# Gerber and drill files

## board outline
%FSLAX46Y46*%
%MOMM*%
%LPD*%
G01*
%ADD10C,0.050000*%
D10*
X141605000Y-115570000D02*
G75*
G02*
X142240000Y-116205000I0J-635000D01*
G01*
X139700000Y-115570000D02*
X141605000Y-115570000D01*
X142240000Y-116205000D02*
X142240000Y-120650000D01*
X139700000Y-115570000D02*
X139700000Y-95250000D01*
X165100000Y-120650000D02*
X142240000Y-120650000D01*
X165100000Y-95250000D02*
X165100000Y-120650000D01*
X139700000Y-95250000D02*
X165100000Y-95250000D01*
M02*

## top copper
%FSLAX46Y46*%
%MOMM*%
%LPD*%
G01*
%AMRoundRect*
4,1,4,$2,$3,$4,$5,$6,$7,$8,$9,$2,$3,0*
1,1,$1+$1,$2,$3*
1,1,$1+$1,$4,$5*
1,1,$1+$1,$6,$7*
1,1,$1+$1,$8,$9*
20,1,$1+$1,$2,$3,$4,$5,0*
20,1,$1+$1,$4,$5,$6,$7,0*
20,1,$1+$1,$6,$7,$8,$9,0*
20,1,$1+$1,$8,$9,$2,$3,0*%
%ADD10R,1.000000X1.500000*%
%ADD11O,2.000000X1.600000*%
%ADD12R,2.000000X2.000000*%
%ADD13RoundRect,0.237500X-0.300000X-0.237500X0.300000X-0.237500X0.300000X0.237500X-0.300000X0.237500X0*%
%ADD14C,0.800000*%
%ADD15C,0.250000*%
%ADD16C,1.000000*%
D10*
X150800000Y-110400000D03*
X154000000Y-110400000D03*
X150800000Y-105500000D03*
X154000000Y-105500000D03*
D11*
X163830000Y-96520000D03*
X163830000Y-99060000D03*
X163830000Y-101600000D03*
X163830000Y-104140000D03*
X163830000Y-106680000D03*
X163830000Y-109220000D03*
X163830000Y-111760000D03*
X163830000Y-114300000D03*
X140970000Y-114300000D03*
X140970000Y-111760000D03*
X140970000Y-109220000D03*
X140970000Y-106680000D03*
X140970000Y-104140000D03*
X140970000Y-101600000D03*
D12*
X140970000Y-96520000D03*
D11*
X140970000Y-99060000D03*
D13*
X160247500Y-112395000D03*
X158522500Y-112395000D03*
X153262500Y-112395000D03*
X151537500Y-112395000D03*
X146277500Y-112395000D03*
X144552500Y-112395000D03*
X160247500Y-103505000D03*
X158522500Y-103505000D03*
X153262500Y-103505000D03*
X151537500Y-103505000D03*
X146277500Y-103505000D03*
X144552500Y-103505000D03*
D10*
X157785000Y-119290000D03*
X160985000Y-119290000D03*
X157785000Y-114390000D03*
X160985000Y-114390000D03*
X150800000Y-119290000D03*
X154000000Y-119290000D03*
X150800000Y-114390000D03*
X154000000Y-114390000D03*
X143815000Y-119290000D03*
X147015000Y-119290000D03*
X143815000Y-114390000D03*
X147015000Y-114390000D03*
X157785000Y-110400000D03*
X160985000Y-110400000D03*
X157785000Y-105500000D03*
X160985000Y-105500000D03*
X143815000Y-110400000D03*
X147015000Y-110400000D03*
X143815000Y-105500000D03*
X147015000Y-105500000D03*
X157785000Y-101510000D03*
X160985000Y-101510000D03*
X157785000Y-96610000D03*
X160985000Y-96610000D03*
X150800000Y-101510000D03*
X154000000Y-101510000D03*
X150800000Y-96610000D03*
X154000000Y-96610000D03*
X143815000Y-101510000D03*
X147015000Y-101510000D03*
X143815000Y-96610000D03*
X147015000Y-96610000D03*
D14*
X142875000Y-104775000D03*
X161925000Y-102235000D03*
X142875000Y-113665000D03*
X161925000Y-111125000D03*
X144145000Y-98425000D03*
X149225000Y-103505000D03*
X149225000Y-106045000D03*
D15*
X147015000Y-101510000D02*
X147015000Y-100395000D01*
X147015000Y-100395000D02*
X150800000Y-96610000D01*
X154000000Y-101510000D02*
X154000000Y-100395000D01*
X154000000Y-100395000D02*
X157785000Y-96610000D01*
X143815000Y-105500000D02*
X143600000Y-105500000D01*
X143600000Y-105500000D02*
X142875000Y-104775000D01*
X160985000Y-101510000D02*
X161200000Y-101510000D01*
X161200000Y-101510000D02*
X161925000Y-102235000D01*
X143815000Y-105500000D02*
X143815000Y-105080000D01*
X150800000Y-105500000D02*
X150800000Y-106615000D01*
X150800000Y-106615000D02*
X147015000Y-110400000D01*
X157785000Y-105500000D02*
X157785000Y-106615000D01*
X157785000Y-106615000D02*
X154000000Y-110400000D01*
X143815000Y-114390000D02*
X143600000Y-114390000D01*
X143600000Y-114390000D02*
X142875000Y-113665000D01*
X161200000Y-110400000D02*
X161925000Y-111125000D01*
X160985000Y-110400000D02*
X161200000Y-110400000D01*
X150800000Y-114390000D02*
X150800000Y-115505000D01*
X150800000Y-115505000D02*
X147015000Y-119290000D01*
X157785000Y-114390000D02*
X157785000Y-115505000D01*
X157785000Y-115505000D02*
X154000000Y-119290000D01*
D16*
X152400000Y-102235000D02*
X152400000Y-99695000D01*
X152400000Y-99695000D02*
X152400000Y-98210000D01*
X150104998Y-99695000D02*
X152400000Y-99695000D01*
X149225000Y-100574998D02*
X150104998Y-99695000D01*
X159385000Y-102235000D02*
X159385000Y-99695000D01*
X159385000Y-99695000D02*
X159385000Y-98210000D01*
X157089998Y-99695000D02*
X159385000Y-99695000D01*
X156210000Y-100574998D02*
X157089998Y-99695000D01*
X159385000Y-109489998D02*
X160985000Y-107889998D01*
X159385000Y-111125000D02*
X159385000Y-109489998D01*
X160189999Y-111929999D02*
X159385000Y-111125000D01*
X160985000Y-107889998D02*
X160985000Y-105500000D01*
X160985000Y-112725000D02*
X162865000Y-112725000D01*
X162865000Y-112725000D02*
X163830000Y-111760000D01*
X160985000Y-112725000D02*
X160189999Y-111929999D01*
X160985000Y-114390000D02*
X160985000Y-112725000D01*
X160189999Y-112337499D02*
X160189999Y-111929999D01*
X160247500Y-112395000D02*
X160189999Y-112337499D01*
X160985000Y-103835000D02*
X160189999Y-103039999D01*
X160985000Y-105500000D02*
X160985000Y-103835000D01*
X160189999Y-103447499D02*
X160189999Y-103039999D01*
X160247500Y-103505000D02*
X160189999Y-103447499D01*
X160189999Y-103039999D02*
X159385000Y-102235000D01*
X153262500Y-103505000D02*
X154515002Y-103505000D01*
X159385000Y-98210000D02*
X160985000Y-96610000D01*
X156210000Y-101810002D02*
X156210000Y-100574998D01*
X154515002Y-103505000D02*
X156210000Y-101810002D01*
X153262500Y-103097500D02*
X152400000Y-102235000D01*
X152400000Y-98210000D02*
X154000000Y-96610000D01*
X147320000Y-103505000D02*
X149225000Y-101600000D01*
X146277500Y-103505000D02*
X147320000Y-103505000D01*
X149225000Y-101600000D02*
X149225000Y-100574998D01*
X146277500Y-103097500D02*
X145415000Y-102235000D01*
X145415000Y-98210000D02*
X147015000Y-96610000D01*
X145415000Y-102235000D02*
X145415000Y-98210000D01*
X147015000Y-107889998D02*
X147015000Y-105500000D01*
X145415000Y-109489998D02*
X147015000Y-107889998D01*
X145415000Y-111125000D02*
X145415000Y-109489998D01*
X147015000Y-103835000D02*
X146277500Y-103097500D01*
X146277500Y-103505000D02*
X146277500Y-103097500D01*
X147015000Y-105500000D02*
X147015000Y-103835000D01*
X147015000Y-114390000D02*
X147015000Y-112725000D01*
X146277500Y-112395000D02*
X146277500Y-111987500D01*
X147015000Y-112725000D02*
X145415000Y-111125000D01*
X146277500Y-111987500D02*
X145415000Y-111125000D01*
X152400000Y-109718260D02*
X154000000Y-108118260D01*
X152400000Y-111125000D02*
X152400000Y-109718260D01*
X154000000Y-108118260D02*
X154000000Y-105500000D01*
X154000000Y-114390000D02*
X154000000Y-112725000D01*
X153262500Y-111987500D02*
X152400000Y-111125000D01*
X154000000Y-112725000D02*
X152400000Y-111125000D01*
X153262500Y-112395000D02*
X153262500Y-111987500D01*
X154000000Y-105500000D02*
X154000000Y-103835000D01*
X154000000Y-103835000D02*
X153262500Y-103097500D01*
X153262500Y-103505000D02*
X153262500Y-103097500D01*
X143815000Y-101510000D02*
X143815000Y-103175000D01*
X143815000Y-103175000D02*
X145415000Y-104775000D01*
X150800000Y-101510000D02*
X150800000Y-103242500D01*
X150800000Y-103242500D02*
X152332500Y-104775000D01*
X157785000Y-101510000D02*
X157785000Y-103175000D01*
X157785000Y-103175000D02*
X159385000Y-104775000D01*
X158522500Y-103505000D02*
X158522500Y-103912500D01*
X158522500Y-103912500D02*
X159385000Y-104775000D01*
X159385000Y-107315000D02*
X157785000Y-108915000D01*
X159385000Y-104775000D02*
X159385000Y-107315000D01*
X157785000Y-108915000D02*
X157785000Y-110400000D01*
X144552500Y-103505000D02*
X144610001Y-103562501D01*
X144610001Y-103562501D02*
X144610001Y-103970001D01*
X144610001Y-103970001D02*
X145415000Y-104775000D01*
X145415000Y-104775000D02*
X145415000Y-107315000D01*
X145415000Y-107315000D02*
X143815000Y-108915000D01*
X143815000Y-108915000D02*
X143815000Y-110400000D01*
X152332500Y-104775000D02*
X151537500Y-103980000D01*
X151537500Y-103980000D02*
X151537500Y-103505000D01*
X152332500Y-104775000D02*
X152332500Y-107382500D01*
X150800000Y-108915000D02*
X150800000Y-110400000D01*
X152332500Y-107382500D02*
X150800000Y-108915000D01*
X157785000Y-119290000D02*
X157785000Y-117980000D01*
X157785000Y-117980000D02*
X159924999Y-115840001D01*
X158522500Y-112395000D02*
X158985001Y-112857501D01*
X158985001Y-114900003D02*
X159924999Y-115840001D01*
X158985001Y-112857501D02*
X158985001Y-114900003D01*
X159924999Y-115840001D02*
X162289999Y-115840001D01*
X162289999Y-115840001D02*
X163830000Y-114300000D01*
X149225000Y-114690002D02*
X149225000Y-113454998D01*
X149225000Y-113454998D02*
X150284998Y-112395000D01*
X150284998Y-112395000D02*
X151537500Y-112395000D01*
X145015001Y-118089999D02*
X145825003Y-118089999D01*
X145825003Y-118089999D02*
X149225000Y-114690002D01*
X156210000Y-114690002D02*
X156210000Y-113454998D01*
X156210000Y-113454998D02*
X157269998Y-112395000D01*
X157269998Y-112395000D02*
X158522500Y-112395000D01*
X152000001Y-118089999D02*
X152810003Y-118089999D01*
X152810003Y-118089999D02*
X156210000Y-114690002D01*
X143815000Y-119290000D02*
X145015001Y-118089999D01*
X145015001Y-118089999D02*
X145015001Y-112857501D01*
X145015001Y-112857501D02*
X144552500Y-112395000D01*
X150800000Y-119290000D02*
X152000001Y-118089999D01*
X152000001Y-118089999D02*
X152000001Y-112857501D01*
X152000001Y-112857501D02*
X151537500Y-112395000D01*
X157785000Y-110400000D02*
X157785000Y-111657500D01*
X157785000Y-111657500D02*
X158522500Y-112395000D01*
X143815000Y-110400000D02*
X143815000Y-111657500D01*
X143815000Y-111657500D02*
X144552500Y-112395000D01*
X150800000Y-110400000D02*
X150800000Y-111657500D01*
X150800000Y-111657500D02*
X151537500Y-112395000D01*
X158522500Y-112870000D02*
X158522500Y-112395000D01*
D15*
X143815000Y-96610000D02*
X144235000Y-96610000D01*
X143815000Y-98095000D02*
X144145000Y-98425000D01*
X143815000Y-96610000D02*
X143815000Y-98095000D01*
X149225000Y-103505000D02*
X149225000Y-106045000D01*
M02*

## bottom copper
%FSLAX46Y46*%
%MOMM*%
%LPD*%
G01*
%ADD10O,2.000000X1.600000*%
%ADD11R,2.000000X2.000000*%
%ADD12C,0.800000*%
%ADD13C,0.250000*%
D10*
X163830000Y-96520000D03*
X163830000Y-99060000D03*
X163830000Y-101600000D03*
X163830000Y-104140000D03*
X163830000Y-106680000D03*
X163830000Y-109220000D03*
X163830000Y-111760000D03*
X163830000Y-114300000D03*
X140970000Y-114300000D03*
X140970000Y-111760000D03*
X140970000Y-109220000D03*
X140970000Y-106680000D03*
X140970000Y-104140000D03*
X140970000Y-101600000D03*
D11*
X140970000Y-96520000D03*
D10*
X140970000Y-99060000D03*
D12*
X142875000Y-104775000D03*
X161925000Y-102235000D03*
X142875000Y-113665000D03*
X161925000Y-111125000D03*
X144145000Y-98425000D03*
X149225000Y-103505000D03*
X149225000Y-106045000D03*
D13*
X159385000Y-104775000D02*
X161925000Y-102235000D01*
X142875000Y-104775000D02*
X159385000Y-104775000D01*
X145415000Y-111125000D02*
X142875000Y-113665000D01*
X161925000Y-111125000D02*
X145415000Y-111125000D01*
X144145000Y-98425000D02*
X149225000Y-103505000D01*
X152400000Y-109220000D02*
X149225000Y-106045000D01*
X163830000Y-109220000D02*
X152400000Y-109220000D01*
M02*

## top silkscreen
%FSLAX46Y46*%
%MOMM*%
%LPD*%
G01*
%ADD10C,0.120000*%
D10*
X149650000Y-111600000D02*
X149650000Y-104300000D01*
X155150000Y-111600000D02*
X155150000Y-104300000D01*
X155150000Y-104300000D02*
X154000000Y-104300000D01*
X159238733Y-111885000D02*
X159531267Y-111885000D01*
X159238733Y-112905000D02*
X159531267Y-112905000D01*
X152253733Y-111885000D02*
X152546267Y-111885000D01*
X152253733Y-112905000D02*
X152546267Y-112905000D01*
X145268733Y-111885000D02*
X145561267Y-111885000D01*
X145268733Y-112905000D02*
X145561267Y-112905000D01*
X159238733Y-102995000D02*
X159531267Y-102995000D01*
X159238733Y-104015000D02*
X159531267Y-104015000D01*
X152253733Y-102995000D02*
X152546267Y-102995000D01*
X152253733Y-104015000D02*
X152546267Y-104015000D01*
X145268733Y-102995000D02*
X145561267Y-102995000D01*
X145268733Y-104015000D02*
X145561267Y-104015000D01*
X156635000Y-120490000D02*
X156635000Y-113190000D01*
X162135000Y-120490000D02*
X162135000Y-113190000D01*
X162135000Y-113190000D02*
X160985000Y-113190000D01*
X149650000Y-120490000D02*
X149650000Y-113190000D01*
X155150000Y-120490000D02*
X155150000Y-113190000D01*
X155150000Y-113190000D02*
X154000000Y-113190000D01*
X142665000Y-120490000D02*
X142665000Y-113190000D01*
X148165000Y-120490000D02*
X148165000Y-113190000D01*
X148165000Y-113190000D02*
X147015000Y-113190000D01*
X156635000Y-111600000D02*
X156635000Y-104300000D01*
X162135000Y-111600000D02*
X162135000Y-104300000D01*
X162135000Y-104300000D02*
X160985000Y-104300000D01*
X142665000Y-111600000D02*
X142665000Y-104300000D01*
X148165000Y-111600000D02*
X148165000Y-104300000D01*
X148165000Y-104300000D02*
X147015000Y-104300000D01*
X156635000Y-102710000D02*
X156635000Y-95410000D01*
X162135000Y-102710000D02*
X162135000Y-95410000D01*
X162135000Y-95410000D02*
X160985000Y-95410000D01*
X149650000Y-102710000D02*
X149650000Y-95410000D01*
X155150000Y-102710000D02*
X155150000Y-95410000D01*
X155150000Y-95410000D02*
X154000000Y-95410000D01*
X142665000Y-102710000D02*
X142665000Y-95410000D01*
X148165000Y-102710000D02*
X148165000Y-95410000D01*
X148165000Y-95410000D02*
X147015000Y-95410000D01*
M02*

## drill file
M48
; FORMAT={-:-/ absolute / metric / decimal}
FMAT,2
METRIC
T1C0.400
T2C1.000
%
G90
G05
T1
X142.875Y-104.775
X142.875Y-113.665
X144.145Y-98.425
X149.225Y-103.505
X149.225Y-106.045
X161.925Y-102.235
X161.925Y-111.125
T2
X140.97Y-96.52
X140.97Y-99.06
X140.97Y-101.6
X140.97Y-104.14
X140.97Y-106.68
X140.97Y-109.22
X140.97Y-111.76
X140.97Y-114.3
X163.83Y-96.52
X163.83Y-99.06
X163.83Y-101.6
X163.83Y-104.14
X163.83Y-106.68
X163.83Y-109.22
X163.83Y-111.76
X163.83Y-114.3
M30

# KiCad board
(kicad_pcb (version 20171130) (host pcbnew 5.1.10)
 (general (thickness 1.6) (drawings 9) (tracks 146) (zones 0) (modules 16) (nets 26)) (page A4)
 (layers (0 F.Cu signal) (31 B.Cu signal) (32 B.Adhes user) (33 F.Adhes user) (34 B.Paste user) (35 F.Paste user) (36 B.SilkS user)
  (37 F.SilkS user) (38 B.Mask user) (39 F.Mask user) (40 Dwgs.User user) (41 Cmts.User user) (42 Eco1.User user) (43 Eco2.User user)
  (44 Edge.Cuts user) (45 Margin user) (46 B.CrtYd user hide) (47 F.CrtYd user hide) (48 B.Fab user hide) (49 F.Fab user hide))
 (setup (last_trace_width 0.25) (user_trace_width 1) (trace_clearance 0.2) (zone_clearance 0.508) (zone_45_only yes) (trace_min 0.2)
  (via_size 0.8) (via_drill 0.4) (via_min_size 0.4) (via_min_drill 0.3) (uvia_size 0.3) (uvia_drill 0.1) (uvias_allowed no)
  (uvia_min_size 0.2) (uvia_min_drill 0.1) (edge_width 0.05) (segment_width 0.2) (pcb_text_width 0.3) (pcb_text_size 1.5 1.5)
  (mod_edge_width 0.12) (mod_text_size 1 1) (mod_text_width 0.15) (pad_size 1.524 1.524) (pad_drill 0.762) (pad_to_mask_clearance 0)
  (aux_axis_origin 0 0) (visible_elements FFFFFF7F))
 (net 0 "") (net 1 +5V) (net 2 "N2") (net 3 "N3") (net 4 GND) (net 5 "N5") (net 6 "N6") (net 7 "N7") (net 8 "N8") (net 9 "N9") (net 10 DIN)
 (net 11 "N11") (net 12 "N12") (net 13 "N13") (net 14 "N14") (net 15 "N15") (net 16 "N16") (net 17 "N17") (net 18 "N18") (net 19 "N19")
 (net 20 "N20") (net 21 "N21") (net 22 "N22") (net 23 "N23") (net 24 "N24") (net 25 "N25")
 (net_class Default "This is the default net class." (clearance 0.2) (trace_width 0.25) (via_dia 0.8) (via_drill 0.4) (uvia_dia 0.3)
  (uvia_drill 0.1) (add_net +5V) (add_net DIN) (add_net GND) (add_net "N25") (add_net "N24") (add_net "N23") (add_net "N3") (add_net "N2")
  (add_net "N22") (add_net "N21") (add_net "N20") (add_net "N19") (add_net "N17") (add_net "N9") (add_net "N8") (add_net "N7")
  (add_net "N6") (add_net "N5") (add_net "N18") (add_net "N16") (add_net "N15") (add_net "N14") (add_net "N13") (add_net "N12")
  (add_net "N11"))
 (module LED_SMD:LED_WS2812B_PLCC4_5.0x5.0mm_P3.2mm (layer F.Cu) (at 152.4 107.95 90)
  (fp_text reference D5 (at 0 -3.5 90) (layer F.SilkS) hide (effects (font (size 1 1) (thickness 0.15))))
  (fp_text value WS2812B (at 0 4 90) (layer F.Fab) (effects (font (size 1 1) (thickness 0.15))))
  (fp_line (start -3.65 -2.75) (end 3.65 -2.75) (layer F.SilkS) (width 0.12))
  (fp_line (start -3.65 2.75) (end 3.65 2.75) (layer F.SilkS) (width 0.12))
  (fp_line (start 3.65 2.75) (end 3.65 1.6) (layer F.SilkS) (width 0.12))
  (pad 1 smd rect (at -2.45 -1.6 90) (size 1.5 1) (layers F.Cu F.Paste F.Mask) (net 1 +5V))
  (pad 2 smd rect (at -2.45 1.6 90) (size 1.5 1) (layers F.Cu F.Paste F.Mask) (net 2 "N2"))
  (pad 4 smd rect (at 2.45 -1.6 90) (size 1.5 1) (layers F.Cu F.Paste F.Mask) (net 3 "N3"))
  (pad 3 smd rect (at 2.45 1.6 90) (size 1.5 1) (layers F.Cu F.Paste F.Mask) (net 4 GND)))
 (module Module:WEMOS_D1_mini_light (layer F.Cu) (at 140.97 96.52)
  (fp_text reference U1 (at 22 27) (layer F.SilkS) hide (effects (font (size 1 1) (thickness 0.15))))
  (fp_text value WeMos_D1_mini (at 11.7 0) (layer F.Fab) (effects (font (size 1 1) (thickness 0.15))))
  (pad 16 thru_hole oval (at 22.86 0) (size 2 1.6) (drill 1) (layers *.Cu *.Mask) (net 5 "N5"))
  (pad 15 thru_hole oval (at 22.86 2.54) (size 2 1.6) (drill 1) (layers *.Cu *.Mask) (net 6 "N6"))
  (pad 14 thru_hole oval (at 22.86 5.08) (size 2 1.6) (drill 1) (layers *.Cu *.Mask) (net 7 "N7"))
  (pad 13 thru_hole oval (at 22.86 7.62) (size 2 1.6) (drill 1) (layers *.Cu *.Mask) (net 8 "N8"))
  (pad 12 thru_hole oval (at 22.86 10.16) (size 2 1.6) (drill 1) (layers *.Cu *.Mask) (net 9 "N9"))
  (pad 11 thru_hole oval (at 22.86 12.7) (size 2 1.6) (drill 1) (layers *.Cu *.Mask) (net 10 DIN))
  (pad 10 thru_hole oval (at 22.86 15.24) (size 2 1.6) (drill 1) (layers *.Cu *.Mask) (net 4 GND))
  (pad 9 thru_hole oval (at 22.86 17.78) (size 2 1.6) (drill 1) (layers *.Cu *.Mask) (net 1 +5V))
  (pad 8 thru_hole oval (at 0 17.78) (size 2 1.6) (drill 1) (layers *.Cu *.Mask) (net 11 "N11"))
  (pad 7 thru_hole oval (at 0 15.24) (size 2 1.6) (drill 1) (layers *.Cu *.Mask) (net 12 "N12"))
  (pad 6 thru_hole oval (at 0 12.7) (size 2 1.6) (drill 1) (layers *.Cu *.Mask) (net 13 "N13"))
  (pad 5 thru_hole oval (at 0 10.16) (size 2 1.6) (drill 1) (layers *.Cu *.Mask) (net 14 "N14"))
  (pad 4 thru_hole oval (at 0 7.62) (size 2 1.6) (drill 1) (layers *.Cu *.Mask) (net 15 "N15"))
  (pad 3 thru_hole oval (at 0 5.08) (size 2 1.6) (drill 1) (layers *.Cu *.Mask) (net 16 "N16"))
  (pad 1 thru_hole rect (at 0 0) (size 2 2) (drill 1) (layers *.Cu *.Mask) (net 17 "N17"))
  (pad 2 thru_hole oval (at 0 2.54) (size 2 1.6) (drill 1) (layers *.Cu *.Mask) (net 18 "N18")))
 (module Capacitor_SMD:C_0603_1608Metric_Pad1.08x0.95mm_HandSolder (layer F.Cu) (at 159.385 112.395)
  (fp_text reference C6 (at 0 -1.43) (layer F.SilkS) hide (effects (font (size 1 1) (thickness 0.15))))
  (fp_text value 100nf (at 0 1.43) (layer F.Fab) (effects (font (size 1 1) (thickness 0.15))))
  (fp_line (start -0.146267 -0.51) (end 0.146267 -0.51) (layer F.SilkS) (width 0.12))
  (fp_line (start -0.146267 0.51) (end 0.146267 0.51) (layer F.SilkS) (width 0.12))
  (pad 2 smd roundrect (at 0.8625 0) (size 1.075 0.95) (layers F.Cu F.Paste F.Mask) (roundrect_rratio 0.25) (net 4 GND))
  (pad 1 smd roundrect (at -0.8625 0) (size 1.075 0.95) (layers F.Cu F.Paste F.Mask) (roundrect_rratio 0.25) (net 1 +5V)))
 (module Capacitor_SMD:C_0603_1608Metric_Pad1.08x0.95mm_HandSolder (layer F.Cu) (at 152.4 112.395)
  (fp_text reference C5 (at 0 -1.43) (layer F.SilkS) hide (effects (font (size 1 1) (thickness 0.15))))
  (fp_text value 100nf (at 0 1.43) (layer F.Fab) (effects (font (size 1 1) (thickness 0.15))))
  (fp_line (start -0.146267 -0.51) (end 0.146267 -0.51) (layer F.SilkS) (width 0.12))
  (fp_line (start -0.146267 0.51) (end 0.146267 0.51) (layer F.SilkS) (width 0.12))
  (pad 2 smd roundrect (at 0.8625 0) (size 1.075 0.95) (layers F.Cu F.Paste F.Mask) (roundrect_rratio 0.25) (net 4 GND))
  (pad 1 smd roundrect (at -0.8625 0) (size 1.075 0.95) (layers F.Cu F.Paste F.Mask) (roundrect_rratio 0.25) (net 1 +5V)))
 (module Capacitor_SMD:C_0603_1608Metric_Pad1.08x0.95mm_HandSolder (layer F.Cu) (at 145.415 112.395)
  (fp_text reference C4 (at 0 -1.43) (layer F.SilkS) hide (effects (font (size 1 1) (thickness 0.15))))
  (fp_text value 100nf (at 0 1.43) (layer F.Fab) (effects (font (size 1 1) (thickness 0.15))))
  (fp_line (start -0.146267 -0.51) (end 0.146267 -0.51) (layer F.SilkS) (width 0.12))
  (fp_line (start -0.146267 0.51) (end 0.146267 0.51) (layer F.SilkS) (width 0.12))
  (pad 2 smd roundrect (at 0.8625 0) (size 1.075 0.95) (layers F.Cu F.Paste F.Mask) (roundrect_rratio 0.25) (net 4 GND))
  (pad 1 smd roundrect (at -0.8625 0) (size 1.075 0.95) (layers F.Cu F.Paste F.Mask) (roundrect_rratio 0.25) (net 1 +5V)))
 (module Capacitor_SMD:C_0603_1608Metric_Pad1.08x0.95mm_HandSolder (layer F.Cu) (at 159.385 103.505)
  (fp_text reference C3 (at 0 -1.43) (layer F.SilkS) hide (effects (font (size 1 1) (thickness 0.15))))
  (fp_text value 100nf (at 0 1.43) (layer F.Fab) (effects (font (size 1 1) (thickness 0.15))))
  (fp_line (start -0.146267 -0.51) (end 0.146267 -0.51) (layer F.SilkS) (width 0.12))
  (fp_line (start -0.146267 0.51) (end 0.146267 0.51) (layer F.SilkS) (width 0.12))
  (pad 2 smd roundrect (at 0.8625 0) (size 1.075 0.95) (layers F.Cu F.Paste F.Mask) (roundrect_rratio 0.25) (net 4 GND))
  (pad 1 smd roundrect (at -0.8625 0) (size 1.075 0.95) (layers F.Cu F.Paste F.Mask) (roundrect_rratio 0.25) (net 1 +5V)))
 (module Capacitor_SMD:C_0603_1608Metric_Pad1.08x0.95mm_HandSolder (layer F.Cu) (at 152.4 103.505)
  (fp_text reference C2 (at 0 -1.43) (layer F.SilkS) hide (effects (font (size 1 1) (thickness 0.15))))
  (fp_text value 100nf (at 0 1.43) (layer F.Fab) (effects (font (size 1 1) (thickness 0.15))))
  (fp_line (start -0.146267 -0.51) (end 0.146267 -0.51) (layer F.SilkS) (width 0.12))
  (fp_line (start -0.146267 0.51) (end 0.146267 0.51) (layer F.SilkS) (width 0.12))
  (pad 2 smd roundrect (at 0.8625 0) (size 1.075 0.95) (layers F.Cu F.Paste F.Mask) (roundrect_rratio 0.25) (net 4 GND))
  (pad 1 smd roundrect (at -0.8625 0) (size 1.075 0.95) (layers F.Cu F.Paste F.Mask) (roundrect_rratio 0.25) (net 1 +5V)))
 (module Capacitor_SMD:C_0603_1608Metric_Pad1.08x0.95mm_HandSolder (layer F.Cu) (at 145.415 103.505)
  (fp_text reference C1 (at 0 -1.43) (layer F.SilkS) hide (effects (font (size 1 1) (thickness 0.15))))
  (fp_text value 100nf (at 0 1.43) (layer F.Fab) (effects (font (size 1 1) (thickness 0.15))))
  (fp_line (start -0.146267 -0.51) (end 0.146267 -0.51) (layer F.SilkS) (width 0.12))
  (fp_line (start -0.146267 0.51) (end 0.146267 0.51) (layer F.SilkS) (width 0.12))
  (pad 2 smd roundrect (at 0.8625 0) (size 1.075 0.95) (layers F.Cu F.Paste F.Mask) (roundrect_rratio 0.25) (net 4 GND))
  (pad 1 smd roundrect (at -0.8625 0) (size 1.075 0.95) (layers F.Cu F.Paste F.Mask) (roundrect_rratio 0.25) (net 1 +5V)))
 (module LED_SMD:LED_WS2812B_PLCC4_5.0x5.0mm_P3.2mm (layer F.Cu) (at 159.385 116.84 90)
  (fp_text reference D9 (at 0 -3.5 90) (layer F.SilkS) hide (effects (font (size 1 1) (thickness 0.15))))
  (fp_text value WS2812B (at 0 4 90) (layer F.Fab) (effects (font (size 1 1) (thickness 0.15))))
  (fp_line (start -3.65 -2.75) (end 3.65 -2.75) (layer F.SilkS) (width 0.12))
  (fp_line (start -3.65 2.75) (end 3.65 2.75) (layer F.SilkS) (width 0.12))
  (fp_line (start 3.65 2.75) (end 3.65 1.6) (layer F.SilkS) (width 0.12))
  (pad 1 smd rect (at -2.45 -1.6 90) (size 1.5 1) (layers F.Cu F.Paste F.Mask) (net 1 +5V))
  (pad 2 smd rect (at -2.45 1.6 90) (size 1.5 1) (layers F.Cu F.Paste F.Mask) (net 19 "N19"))
  (pad 4 smd rect (at 2.45 -1.6 90) (size 1.5 1) (layers F.Cu F.Paste F.Mask) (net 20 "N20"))
  (pad 3 smd rect (at 2.45 1.6 90) (size 1.5 1) (layers F.Cu F.Paste F.Mask) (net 4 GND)))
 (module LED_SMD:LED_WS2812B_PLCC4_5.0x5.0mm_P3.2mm (layer F.Cu) (at 152.4 116.84 90)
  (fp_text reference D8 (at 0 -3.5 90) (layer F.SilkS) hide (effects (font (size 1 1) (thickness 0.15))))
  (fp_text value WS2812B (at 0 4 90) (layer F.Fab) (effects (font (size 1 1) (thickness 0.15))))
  (fp_line (start -3.65 -2.75) (end 3.65 -2.75) (layer F.SilkS) (width 0.12))
  (fp_line (start -3.65 2.75) (end 3.65 2.75) (layer F.SilkS) (width 0.12))
  (fp_line (start 3.65 2.75) (end 3.65 1.6) (layer F.SilkS) (width 0.12))
  (pad 1 smd rect (at -2.45 -1.6 90) (size 1.5 1) (layers F.Cu F.Paste F.Mask) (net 1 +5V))
  (pad 2 smd rect (at -2.45 1.6 90) (size 1.5 1) (layers F.Cu F.Paste F.Mask) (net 20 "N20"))
  (pad 4 smd rect (at 2.45 -1.6 90) (size 1.5 1) (layers F.Cu F.Paste F.Mask) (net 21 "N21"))
  (pad 3 smd rect (at 2.45 1.6 90) (size 1.5 1) (layers F.Cu F.Paste F.Mask) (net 4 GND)))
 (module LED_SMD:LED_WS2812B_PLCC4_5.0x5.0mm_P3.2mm (layer F.Cu) (at 145.415 116.84 90)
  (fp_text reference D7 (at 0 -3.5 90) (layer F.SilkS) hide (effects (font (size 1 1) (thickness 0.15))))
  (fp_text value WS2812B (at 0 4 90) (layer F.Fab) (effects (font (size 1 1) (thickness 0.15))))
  (fp_line (start -3.65 -2.75) (end 3.65 -2.75) (layer F.SilkS) (width 0.12))
  (fp_line (start -3.65 2.75) (end 3.65 2.75) (layer F.SilkS) (width 0.12))
  (fp_line (start 3.65 2.75) (end 3.65 1.6) (layer F.SilkS) (width 0.12))
  (pad 1 smd rect (at -2.45 -1.6 90) (size 1.5 1) (layers F.Cu F.Paste F.Mask) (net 1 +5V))
  (pad 2 smd rect (at -2.45 1.6 90) (size 1.5 1) (layers F.Cu F.Paste F.Mask) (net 21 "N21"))
  (pad 4 smd rect (at 2.45 -1.6 90) (size 1.5 1) (layers F.Cu F.Paste F.Mask) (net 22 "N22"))
  (pad 3 smd rect (at 2.45 1.6 90) (size 1.5 1) (layers F.Cu F.Paste F.Mask) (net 4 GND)))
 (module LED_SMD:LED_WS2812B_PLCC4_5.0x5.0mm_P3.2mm (layer F.Cu) (at 159.385 107.95 90)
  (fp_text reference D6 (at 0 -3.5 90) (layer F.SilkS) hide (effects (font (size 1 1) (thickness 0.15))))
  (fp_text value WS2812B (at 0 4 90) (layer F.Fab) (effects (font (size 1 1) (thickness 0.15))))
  (fp_line (start -3.65 -2.75) (end 3.65 -2.75) (layer F.SilkS) (width 0.12))
  (fp_line (start -3.65 2.75) (end 3.65 2.75) (layer F.SilkS) (width 0.12))
  (fp_line (start 3.65 2.75) (end 3.65 1.6) (layer F.SilkS) (width 0.12))
  (pad 1 smd rect (at -2.45 -1.6 90) (size 1.5 1) (layers F.Cu F.Paste F.Mask) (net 1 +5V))
  (pad 2 smd rect (at -2.45 1.6 90) (size 1.5 1) (layers F.Cu F.Paste F.Mask) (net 22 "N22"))
  (pad 4 smd rect (at 2.45 -1.6 90) (size 1.5 1) (layers F.Cu F.Paste F.Mask) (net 2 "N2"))
  (pad 3 smd rect (at 2.45 1.6 90) (size 1.5 1) (layers F.Cu F.Paste F.Mask) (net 4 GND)))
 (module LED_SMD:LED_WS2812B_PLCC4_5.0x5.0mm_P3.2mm (layer F.Cu) (at 145.415 107.95 90)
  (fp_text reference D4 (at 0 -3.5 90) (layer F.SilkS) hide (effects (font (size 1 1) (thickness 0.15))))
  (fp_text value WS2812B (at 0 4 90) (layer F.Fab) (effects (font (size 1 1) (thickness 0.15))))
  (fp_line (start -3.65 -2.75) (end 3.65 -2.75) (layer F.SilkS) (width 0.12))
  (fp_line (start -3.65 2.75) (end 3.65 2.75) (layer F.SilkS) (width 0.12))
  (fp_line (start 3.65 2.75) (end 3.65 1.6) (layer F.SilkS) (width 0.12))
  (pad 1 smd rect (at -2.45 -1.6 90) (size 1.5 1) (layers F.Cu F.Paste F.Mask) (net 1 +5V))
  (pad 2 smd rect (at -2.45 1.6 90) (size 1.5 1) (layers F.Cu F.Paste F.Mask) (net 3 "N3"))
  (pad 4 smd rect (at 2.45 -1.6 90) (size 1.5 1) (layers F.Cu F.Paste F.Mask) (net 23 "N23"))
  (pad 3 smd rect (at 2.45 1.6 90) (size 1.5 1) (layers F.Cu F.Paste F.Mask) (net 4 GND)))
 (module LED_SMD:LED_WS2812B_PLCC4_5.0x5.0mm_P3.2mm (layer F.Cu) (at 159.385 99.06 90)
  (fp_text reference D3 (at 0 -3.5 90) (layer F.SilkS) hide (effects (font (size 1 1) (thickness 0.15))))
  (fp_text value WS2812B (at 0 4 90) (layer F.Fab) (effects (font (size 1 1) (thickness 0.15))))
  (fp_line (start -3.65 -2.75) (end 3.65 -2.75) (layer F.SilkS) (width 0.12))
  (fp_line (start -3.65 2.75) (end 3.65 2.75) (layer F.SilkS) (width 0.12))
  (fp_line (start 3.65 2.75) (end 3.65 1.6) (layer F.SilkS) (width 0.12))
  (pad 1 smd rect (at -2.45 -1.6 90) (size 1.5 1) (layers F.Cu F.Paste F.Mask) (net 1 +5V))
  (pad 2 smd rect (at -2.45 1.6 90) (size 1.5 1) (layers F.Cu F.Paste F.Mask) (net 23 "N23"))
  (pad 4 smd rect (at 2.45 -1.6 90) (size 1.5 1) (layers F.Cu F.Paste F.Mask) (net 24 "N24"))
  (pad 3 smd rect (at 2.45 1.6 90) (size 1.5 1) (layers F.Cu F.Paste F.Mask) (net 4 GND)))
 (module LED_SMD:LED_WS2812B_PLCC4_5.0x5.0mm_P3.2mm (layer F.Cu) (at 152.4 99.06 90)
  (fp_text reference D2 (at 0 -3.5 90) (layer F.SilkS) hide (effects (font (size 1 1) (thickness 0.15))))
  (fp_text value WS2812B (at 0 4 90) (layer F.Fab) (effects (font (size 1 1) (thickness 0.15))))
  (fp_line (start -3.65 -2.75) (end 3.65 -2.75) (layer F.SilkS) (width 0.12))
  (fp_line (start -3.65 2.75) (end 3.65 2.75) (layer F.SilkS) (width 0.12))
  (fp_line (start 3.65 2.75) (end 3.65 1.6) (layer F.SilkS) (width 0.12))
  (pad 1 smd rect (at -2.45 -1.6 90) (size 1.5 1) (layers F.Cu F.Paste F.Mask) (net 1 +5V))
  (pad 2 smd rect (at -2.45 1.6 90) (size 1.5 1) (layers F.Cu F.Paste F.Mask) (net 24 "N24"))
  (pad 4 smd rect (at 2.45 -1.6 90) (size 1.5 1) (layers F.Cu F.Paste F.Mask) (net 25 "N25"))
  (pad 3 smd rect (at 2.45 1.6 90) (size 1.5 1) (layers F.Cu F.Paste F.Mask) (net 4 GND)))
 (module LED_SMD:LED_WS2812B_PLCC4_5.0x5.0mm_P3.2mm (layer F.Cu) (at 145.415 99.06 90)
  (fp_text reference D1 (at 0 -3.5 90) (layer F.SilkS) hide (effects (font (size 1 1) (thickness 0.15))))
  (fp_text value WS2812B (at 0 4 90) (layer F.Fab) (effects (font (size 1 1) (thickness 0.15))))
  (fp_line (start -3.65 -2.75) (end 3.65 -2.75) (layer F.SilkS) (width 0.12))
  (fp_line (start -3.65 2.75) (end 3.65 2.75) (layer F.SilkS) (width 0.12))
  (fp_line (start 3.65 2.75) (end 3.65 1.6) (layer F.SilkS) (width 0.12))
  (pad 1 smd rect (at -2.45 -1.6 90) (size 1.5 1) (layers F.Cu F.Paste F.Mask) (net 1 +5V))
  (pad 2 smd rect (at -2.45 1.6 90) (size 1.5 1) (layers F.Cu F.Paste F.Mask) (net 25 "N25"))
  (pad 4 smd rect (at 2.45 -1.6 90) (size 1.5 1) (layers F.Cu F.Paste F.Mask) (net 10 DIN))
  (pad 3 smd rect (at 2.45 1.6 90) (size 1.5 1) (layers F.Cu F.Paste F.Mask) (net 4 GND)))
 (gr_arc (start 141.605 116.205) (end 142.24 116.205) (angle -90) (layer Edge.Cuts) (width 0.05))
 (gr_line (start 139.7 115.57) (end 141.605 115.57) (layer Edge.Cuts) (width 0.05))
 (gr_line (start 142.24 116.205) (end 142.24 120.65) (layer Edge.Cuts) (width 0.05))
 (gr_line (start 139.7 115.57) (end 139.7 95.25) (layer Edge.Cuts) (width 0.05))
 (gr_line (start 165.1 120.65) (end 142.24 120.65) (layer Edge.Cuts) (width 0.05))
 (gr_line (start 165.1 95.25) (end 165.1 120.65) (layer Edge.Cuts) (width 0.05))
 (gr_line (start 139.7 95.25) (end 165.1 95.25) (layer Edge.Cuts) (width 0.05))
 (segment (start 147.015 101.51) (end 147.015 100.395) (width 0.25) (layer F.Cu) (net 25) (status 10))
 (segment (start 147.015 100.395) (end 150.8 96.61) (width 0.25) (layer F.Cu) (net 25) (status 20))
 (segment (start 154 101.51) (end 154 100.395) (width 0.25) (layer F.Cu) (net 24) (status 10))
 (segment (start 154 100.395) (end 157.785 96.61) (width 0.25) (layer F.Cu) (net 24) (status 20))
 (segment (start 143.815 105.5) (end 143.6 105.5) (width 0.25) (layer F.Cu) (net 23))
 (segment (start 143.6 105.5) (end 142.875 104.775) (width 0.25) (layer F.Cu) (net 23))
 (via (at 142.875 104.775) (size 0.8) (drill 0.4) (layers F.Cu B.Cu) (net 23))
 (segment (start 160.985 101.51) (end 161.2 101.51) (width 0.25) (layer F.Cu) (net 23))
 (segment (start 161.2 101.51) (end 161.925 102.235) (width 0.25) (layer F.Cu) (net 23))
 (via (at 161.925 102.235) (size 0.8) (drill 0.4) (layers F.Cu B.Cu) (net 23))
 (segment (start 143.815 105.5) (end 143.815 105.08) (width 0.25) (layer F.Cu) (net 23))
 (segment (start 159.385 104.775) (end 161.925 102.235) (width 0.25) (layer B.Cu) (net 23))
 (segment (start 142.875 104.775) (end 159.385 104.775) (width 0.25) (layer B.Cu) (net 23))
 (segment (start 150.8 105.5) (end 150.8 106.615) (width 0.25) (layer F.Cu) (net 3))
 (segment (start 150.8 106.615) (end 147.015 110.4) (width 0.25) (layer F.Cu) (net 3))
 (segment (start 157.785 105.5) (end 157.785 106.615) (width 0.25) (layer F.Cu) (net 2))
 (segment (start 157.785 106.615) (end 154 110.4) (width 0.25) (layer F.Cu) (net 2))
 (segment (start 143.815 114.39) (end 143.6 114.39) (width 0.25) (layer F.Cu) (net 22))
 (via (at 142.875 113.665) (size 0.8) (drill 0.4) (layers F.Cu B.Cu) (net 22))
 (segment (start 143.6 114.39) (end 142.875 113.665) (width 0.25) (layer F.Cu) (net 22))
 (via (at 161.925 111.125) (size 0.8) (drill 0.4) (layers F.Cu B.Cu) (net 22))
 (segment (start 161.2 110.4) (end 161.925 111.125) (width 0.25) (layer F.Cu) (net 22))
 (segment (start 160.985 110.4) (end 161.2 110.4) (width 0.25) (layer F.Cu) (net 22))
 (segment (start 145.415 111.125) (end 142.875 113.665) (width 0.25) (layer B.Cu) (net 22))
 (segment (start 161.925 111.125) (end 145.415 111.125) (width 0.25) (layer B.Cu) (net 22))
 (segment (start 150.8 114.39) (end 150.8 115.505) (width 0.25) (layer F.Cu) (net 21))
 (segment (start 150.8 115.505) (end 147.015 119.29) (width 0.25) (layer F.Cu) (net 21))
 (segment (start 157.785 114.39) (end 157.785 115.505) (width 0.25) (layer F.Cu) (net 20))
 (segment (start 157.785 115.505) (end 154 119.29) (width 0.25) (layer F.Cu) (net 20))
 (segment (start 152.4 102.235) (end 152.4 99.695) (width 1) (layer F.Cu) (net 4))
 (segment (start 152.4 99.695) (end 152.4 98.21) (width 1) (layer F.Cu) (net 4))
 (segment (start 150.104998 99.695) (end 152.4 99.695) (width 1) (layer F.Cu) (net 4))
 (segment (start 149.225 100.574998) (end 150.104998 99.695) (width 1) (layer F.Cu) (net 4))
 (segment (start 159.385 102.235) (end 159.385 99.695) (width 1) (layer F.Cu) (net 4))
 (segment (start 159.385 99.695) (end 159.385 98.21) (width 1) (layer F.Cu) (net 4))
 (segment (start 157.089998 99.695) (end 159.385 99.695) (width 1) (layer F.Cu) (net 4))
 (segment (start 156.21 100.574998) (end 157.089998 99.695) (width 1) (layer F.Cu) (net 4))
 (segment (start 159.385 109.489998) (end 160.985 107.889998) (width 1) (layer F.Cu) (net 4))
 (segment (start 159.385 111.125) (end 159.385 109.489998) (width 1) (layer F.Cu) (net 4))
 (segment (start 160.189999 111.929999) (end 159.385 111.125) (width 1) (layer F.Cu) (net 4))
 (segment (start 160.985 107.889998) (end 160.985 105.5) (width 1) (layer F.Cu) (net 4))
 (segment (start 160.985 112.725) (end 162.865 112.725) (width 1) (layer F.Cu) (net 4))
 (segment (start 162.865 112.725) (end 163.83 111.76) (width 1) (layer F.Cu) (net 4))
 (segment (start 160.985 112.725) (end 160.189999 111.929999) (width 1) (layer F.Cu) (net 4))
 (segment (start 160.985 114.39) (end 160.985 112.725) (width 1) (layer F.Cu) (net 4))
 (segment (start 160.189999 112.337499) (end 160.189999 111.929999) (width 1) (layer F.Cu) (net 4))
 (segment (start 160.2475 112.395) (end 160.189999 112.337499) (width 1) (layer F.Cu) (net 4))
 (segment (start 160.985 103.835) (end 160.189999 103.039999) (width 1) (layer F.Cu) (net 4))
 (segment (start 160.985 105.5) (end 160.985 103.835) (width 1) (layer F.Cu) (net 4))
 (segment (start 160.189999 103.447499) (end 160.189999 103.039999) (width 1) (layer F.Cu) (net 4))
 (segment (start 160.2475 103.505) (end 160.189999 103.447499) (width 1) (layer F.Cu) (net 4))
 (segment (start 160.189999 103.039999) (end 159.385 102.235) (width 1) (layer F.Cu) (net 4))
 (segment (start 153.2625 103.505) (end 154.515002 103.505) (width 1) (layer F.Cu) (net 4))
 (segment (start 159.385 98.21) (end 160.985 96.61) (width 1) (layer F.Cu) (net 4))
 (segment (start 156.21 101.810002) (end 156.21 100.574998) (width 1) (layer F.Cu) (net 4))
 (segment (start 154.515002 103.505) (end 156.21 101.810002) (width 1) (layer F.Cu) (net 4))
 (segment (start 153.2625 103.0975) (end 152.4 102.235) (width 1) (layer F.Cu) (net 4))
 (segment (start 152.4 98.21) (end 154 96.61) (width 1) (layer F.Cu) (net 4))
 (segment (start 147.32 103.505) (end 149.225 101.6) (width 1) (layer F.Cu) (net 4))
 (segment (start 146.2775 103.505) (end 147.32 103.505) (width 1) (layer F.Cu) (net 4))
 (segment (start 149.225 101.6) (end 149.225 100.574998) (width 1) (layer F.Cu) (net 4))
 (segment (start 146.2775 103.0975) (end 145.415 102.235) (width 1) (layer F.Cu) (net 4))
 (segment (start 145.415 98.21) (end 147.015 96.61) (width 1) (layer F.Cu) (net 4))
 (segment (start 145.415 102.235) (end 145.415 98.21) (width 1) (layer F.Cu) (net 4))
 (segment (start 147.015 107.889998) (end 147.015 105.5) (width 1) (layer F.Cu) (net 4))
 (segment (start 145.415 109.489998) (end 147.015 107.889998) (width 1) (layer F.Cu) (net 4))
 (segment (start 145.415 111.125) (end 145.415 109.489998) (width 1) (layer F.Cu) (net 4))
 (segment (start 147.015 103.835) (end 146.2775 103.0975) (width 1) (layer F.Cu) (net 4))
 (segment (start 146.2775 103.505) (end 146.2775 103.0975) (width 1) (layer F.Cu) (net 4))
 (segment (start 147.015 105.5) (end 147.015 103.835) (width 1) (layer F.Cu) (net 4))
 (segment (start 147.015 114.39) (end 147.015 112.725) (width 1) (layer F.Cu) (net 4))
 (segment (start 146.2775 112.395) (end 146.2775 111.9875) (width 1) (layer F.Cu) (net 4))
 (segment (start 147.015 112.725) (end 145.415 111.125) (width 1) (layer F.Cu) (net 4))
 (segment (start 146.2775 111.9875) (end 145.415 111.125) (width 1) (layer F.Cu) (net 4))
 (segment (start 152.4 109.71826) (end 154 108.11826) (width 1) (layer F.Cu) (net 4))
 (segment (start 152.4 111.125) (end 152.4 109.71826) (width 1) (layer F.Cu) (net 4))
 (segment (start 154 108.11826) (end 154 105.5) (width 1) (layer F.Cu) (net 4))
 (segment (start 154 114.39) (end 154 112.725) (width 1) (layer F.Cu) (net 4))
 (segment (start 153.2625 111.9875) (end 152.4 111.125) (width 1) (layer F.Cu) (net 4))
 (segment (start 154 112.725) (end 152.4 111.125) (width 1) (layer F.Cu) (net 4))
 (segment (start 153.2625 112.395) (end 153.2625 111.9875) (width 1) (layer F.Cu) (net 4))
 (segment (start 154 105.5) (end 154 103.835) (width 1) (layer F.Cu) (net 4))
 (segment (start 154 103.835) (end 153.2625 103.0975) (width 1) (layer F.Cu) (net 4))
 (segment (start 153.2625 103.505) (end 153.2625 103.0975) (width 1) (layer F.Cu) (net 4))
 (segment (start 143.815 101.51) (end 143.815 103.175) (width 1) (layer F.Cu) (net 1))
 (segment (start 143.815 103.175) (end 145.415 104.775) (width 1) (layer F.Cu) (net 1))
 (segment (start 150.8 101.51) (end 150.8 103.2425) (width 1) (layer F.Cu) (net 1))
 (segment (start 150.8 103.2425) (end 152.3325 104.775) (width 1) (layer F.Cu) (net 1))
 (segment (start 157.785 101.51) (end 157.785 103.175) (width 1) (layer F.Cu) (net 1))
 (segment (start 157.785 103.175) (end 159.385 104.775) (width 1) (layer F.Cu) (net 1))
 (segment (start 158.5225 103.505) (end 158.5225 103.9125) (width 1) (layer F.Cu) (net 1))
 (segment (start 158.5225 103.9125) (end 159.385 104.775) (width 1) (layer F.Cu) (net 1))
 (segment (start 159.385 107.315) (end 157.785 108.915) (width 1) (layer F.Cu) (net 1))
 (segment (start 159.385 104.775) (end 159.385 107.315) (width 1) (layer F.Cu) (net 1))
 (segment (start 157.785 108.915) (end 157.785 110.4) (width 1) (layer F.Cu) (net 1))
 (segment (start 144.5525 103.505) (end 144.610001 103.562501) (width 1) (layer F.Cu) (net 1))
 (segment (start 144.610001 103.562501) (end 144.610001 103.970001) (width 1) (layer F.Cu) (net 1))
 (segment (start 144.610001 103.970001) (end 145.415 104.775) (width 1) (layer F.Cu) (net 1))
 (segment (start 145.415 104.775) (end 145.415 107.315) (width 1) (layer F.Cu) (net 1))
 (segment (start 145.415 107.315) (end 143.815 108.915) (width 1) (layer F.Cu) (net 1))
 (segment (start 143.815 108.915) (end 143.815 110.4) (width 1) (layer F.Cu) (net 1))
 (segment (start 152.3325 104.775) (end 151.5375 103.98) (width 1) (layer F.Cu) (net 1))
 (segment (start 151.5375 103.98) (end 151.5375 103.505) (width 1) (layer F.Cu) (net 1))
 (segment (start 152.3325 104.775) (end 152.3325 107.3825) (width 1) (layer F.Cu) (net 1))
 (segment (start 150.8 108.915) (end 150.8 110.4) (width 1) (layer F.Cu) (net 1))
 (segment (start 152.3325 107.3825) (end 150.8 108.915) (width 1) (layer F.Cu) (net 1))
 (segment (start 157.785 119.29) (end 157.785 117.98) (width 1) (layer F.Cu) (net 1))
 (segment (start 157.785 117.98) (end 159.924999 115.840001) (width 1) (layer F.Cu) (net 1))
 (segment (start 158.5225 112.395) (end 158.985001 112.857501) (width 1) (layer F.Cu) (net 1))
 (segment (start 158.985001 114.900003) (end 159.924999 115.840001) (width 1) (layer F.Cu) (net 1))
 (segment (start 158.985001 112.857501) (end 158.985001 114.900003) (width 1) (layer F.Cu) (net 1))
 (segment (start 159.924999 115.840001) (end 162.289999 115.840001) (width 1) (layer F.Cu) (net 1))
 (segment (start 162.289999 115.840001) (end 163.83 114.3) (width 1) (layer F.Cu) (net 1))
 (segment (start 149.225 114.690002) (end 149.225 113.454998) (width 1) (layer F.Cu) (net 1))
 (segment (start 149.225 113.454998) (end 150.284998 112.395) (width 1) (layer F.Cu) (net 1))
 (segment (start 150.284998 112.395) (end 151.5375 112.395) (width 1) (layer F.Cu) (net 1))
 (segment (start 145.015001 118.089999) (end 145.825003 118.089999) (width 1) (layer F.Cu) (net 1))
 (segment (start 145.825003 118.089999) (end 149.225 114.690002) (width 1) (layer F.Cu) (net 1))
 (segment (start 156.21 114.690002) (end 156.21 113.454998) (width 1) (layer F.Cu) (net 1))
 (segment (start 156.21 113.454998) (end 157.269998 112.395) (width 1) (layer F.Cu) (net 1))
 (segment (start 157.269998 112.395) (end 158.5225 112.395) (width 1) (layer F.Cu) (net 1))
 (segment (start 152.000001 118.089999) (end 152.810003 118.089999) (width 1) (layer F.Cu) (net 1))
 (segment (start 152.810003 118.089999) (end 156.21 114.690002) (width 1) (layer F.Cu) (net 1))
 (segment (start 143.815 119.29) (end 145.015001 118.089999) (width 1) (layer F.Cu) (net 1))
 (segment (start 145.015001 118.089999) (end 145.015001 112.857501) (width 1) (layer F.Cu) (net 1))
 (segment (start 145.015001 112.857501) (end 144.5525 112.395) (width 1) (layer F.Cu) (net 1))
 (segment (start 150.8 119.29) (end 152.000001 118.089999) (width 1) (layer F.Cu) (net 1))
 (segment (start 152.000001 118.089999) (end 152.000001 112.857501) (width 1) (layer F.Cu) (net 1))
 (segment (start 152.000001 112.857501) (end 151.5375 112.395) (width 1) (layer F.Cu) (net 1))
 (segment (start 157.785 110.4) (end 157.785 111.6575) (width 1) (layer F.Cu) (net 1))
 (segment (start 157.785 111.6575) (end 158.5225 112.395) (width 1) (layer F.Cu) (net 1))
 (segment (start 143.815 110.4) (end 143.815 111.6575) (width 1) (layer F.Cu) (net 1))
 (segment (start 143.815 111.6575) (end 144.5525 112.395) (width 1) (layer F.Cu) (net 1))
 (segment (start 150.8 110.4) (end 150.8 111.6575) (width 1) (layer F.Cu) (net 1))
 (segment (start 150.8 111.6575) (end 151.5375 112.395) (width 1) (layer F.Cu) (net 1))
 (segment (start 158.5225 112.87) (end 158.5225 112.395) (width 1) (layer F.Cu) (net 1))
 (segment (start 143.815 96.61) (end 144.235 96.61) (width 0.25) (layer F.Cu) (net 10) (status 30))
 (via (at 144.145 98.425) (size 0.8) (drill 0.4) (layers F.Cu B.Cu) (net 10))
 (segment (start 143.815 98.095) (end 144.145 98.425) (width 0.25) (layer F.Cu) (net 10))
 (segment (start 143.815 96.61) (end 143.815 98.095) (width 0.25) (layer F.Cu) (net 10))
 (via (at 149.225 103.505) (size 0.8) (drill 0.4) (layers F.Cu B.Cu) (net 10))
 (segment (start 144.145 98.425) (end 149.225 103.505) (width 0.25) (layer B.Cu) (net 10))
 (via (at 149.225 106.045) (size 0.8) (drill 0.4) (layers F.Cu B.Cu) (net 10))
 (segment (start 149.225 103.505) (end 149.225 106.045) (width 0.25) (layer F.Cu) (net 10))
 (segment (start 152.4 109.22) (end 149.225 106.045) (width 0.25) (layer B.Cu) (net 10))
 (segment (start 163.83 109.22) (end 152.4 109.22) (width 0.25) (layer B.Cu) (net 10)))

